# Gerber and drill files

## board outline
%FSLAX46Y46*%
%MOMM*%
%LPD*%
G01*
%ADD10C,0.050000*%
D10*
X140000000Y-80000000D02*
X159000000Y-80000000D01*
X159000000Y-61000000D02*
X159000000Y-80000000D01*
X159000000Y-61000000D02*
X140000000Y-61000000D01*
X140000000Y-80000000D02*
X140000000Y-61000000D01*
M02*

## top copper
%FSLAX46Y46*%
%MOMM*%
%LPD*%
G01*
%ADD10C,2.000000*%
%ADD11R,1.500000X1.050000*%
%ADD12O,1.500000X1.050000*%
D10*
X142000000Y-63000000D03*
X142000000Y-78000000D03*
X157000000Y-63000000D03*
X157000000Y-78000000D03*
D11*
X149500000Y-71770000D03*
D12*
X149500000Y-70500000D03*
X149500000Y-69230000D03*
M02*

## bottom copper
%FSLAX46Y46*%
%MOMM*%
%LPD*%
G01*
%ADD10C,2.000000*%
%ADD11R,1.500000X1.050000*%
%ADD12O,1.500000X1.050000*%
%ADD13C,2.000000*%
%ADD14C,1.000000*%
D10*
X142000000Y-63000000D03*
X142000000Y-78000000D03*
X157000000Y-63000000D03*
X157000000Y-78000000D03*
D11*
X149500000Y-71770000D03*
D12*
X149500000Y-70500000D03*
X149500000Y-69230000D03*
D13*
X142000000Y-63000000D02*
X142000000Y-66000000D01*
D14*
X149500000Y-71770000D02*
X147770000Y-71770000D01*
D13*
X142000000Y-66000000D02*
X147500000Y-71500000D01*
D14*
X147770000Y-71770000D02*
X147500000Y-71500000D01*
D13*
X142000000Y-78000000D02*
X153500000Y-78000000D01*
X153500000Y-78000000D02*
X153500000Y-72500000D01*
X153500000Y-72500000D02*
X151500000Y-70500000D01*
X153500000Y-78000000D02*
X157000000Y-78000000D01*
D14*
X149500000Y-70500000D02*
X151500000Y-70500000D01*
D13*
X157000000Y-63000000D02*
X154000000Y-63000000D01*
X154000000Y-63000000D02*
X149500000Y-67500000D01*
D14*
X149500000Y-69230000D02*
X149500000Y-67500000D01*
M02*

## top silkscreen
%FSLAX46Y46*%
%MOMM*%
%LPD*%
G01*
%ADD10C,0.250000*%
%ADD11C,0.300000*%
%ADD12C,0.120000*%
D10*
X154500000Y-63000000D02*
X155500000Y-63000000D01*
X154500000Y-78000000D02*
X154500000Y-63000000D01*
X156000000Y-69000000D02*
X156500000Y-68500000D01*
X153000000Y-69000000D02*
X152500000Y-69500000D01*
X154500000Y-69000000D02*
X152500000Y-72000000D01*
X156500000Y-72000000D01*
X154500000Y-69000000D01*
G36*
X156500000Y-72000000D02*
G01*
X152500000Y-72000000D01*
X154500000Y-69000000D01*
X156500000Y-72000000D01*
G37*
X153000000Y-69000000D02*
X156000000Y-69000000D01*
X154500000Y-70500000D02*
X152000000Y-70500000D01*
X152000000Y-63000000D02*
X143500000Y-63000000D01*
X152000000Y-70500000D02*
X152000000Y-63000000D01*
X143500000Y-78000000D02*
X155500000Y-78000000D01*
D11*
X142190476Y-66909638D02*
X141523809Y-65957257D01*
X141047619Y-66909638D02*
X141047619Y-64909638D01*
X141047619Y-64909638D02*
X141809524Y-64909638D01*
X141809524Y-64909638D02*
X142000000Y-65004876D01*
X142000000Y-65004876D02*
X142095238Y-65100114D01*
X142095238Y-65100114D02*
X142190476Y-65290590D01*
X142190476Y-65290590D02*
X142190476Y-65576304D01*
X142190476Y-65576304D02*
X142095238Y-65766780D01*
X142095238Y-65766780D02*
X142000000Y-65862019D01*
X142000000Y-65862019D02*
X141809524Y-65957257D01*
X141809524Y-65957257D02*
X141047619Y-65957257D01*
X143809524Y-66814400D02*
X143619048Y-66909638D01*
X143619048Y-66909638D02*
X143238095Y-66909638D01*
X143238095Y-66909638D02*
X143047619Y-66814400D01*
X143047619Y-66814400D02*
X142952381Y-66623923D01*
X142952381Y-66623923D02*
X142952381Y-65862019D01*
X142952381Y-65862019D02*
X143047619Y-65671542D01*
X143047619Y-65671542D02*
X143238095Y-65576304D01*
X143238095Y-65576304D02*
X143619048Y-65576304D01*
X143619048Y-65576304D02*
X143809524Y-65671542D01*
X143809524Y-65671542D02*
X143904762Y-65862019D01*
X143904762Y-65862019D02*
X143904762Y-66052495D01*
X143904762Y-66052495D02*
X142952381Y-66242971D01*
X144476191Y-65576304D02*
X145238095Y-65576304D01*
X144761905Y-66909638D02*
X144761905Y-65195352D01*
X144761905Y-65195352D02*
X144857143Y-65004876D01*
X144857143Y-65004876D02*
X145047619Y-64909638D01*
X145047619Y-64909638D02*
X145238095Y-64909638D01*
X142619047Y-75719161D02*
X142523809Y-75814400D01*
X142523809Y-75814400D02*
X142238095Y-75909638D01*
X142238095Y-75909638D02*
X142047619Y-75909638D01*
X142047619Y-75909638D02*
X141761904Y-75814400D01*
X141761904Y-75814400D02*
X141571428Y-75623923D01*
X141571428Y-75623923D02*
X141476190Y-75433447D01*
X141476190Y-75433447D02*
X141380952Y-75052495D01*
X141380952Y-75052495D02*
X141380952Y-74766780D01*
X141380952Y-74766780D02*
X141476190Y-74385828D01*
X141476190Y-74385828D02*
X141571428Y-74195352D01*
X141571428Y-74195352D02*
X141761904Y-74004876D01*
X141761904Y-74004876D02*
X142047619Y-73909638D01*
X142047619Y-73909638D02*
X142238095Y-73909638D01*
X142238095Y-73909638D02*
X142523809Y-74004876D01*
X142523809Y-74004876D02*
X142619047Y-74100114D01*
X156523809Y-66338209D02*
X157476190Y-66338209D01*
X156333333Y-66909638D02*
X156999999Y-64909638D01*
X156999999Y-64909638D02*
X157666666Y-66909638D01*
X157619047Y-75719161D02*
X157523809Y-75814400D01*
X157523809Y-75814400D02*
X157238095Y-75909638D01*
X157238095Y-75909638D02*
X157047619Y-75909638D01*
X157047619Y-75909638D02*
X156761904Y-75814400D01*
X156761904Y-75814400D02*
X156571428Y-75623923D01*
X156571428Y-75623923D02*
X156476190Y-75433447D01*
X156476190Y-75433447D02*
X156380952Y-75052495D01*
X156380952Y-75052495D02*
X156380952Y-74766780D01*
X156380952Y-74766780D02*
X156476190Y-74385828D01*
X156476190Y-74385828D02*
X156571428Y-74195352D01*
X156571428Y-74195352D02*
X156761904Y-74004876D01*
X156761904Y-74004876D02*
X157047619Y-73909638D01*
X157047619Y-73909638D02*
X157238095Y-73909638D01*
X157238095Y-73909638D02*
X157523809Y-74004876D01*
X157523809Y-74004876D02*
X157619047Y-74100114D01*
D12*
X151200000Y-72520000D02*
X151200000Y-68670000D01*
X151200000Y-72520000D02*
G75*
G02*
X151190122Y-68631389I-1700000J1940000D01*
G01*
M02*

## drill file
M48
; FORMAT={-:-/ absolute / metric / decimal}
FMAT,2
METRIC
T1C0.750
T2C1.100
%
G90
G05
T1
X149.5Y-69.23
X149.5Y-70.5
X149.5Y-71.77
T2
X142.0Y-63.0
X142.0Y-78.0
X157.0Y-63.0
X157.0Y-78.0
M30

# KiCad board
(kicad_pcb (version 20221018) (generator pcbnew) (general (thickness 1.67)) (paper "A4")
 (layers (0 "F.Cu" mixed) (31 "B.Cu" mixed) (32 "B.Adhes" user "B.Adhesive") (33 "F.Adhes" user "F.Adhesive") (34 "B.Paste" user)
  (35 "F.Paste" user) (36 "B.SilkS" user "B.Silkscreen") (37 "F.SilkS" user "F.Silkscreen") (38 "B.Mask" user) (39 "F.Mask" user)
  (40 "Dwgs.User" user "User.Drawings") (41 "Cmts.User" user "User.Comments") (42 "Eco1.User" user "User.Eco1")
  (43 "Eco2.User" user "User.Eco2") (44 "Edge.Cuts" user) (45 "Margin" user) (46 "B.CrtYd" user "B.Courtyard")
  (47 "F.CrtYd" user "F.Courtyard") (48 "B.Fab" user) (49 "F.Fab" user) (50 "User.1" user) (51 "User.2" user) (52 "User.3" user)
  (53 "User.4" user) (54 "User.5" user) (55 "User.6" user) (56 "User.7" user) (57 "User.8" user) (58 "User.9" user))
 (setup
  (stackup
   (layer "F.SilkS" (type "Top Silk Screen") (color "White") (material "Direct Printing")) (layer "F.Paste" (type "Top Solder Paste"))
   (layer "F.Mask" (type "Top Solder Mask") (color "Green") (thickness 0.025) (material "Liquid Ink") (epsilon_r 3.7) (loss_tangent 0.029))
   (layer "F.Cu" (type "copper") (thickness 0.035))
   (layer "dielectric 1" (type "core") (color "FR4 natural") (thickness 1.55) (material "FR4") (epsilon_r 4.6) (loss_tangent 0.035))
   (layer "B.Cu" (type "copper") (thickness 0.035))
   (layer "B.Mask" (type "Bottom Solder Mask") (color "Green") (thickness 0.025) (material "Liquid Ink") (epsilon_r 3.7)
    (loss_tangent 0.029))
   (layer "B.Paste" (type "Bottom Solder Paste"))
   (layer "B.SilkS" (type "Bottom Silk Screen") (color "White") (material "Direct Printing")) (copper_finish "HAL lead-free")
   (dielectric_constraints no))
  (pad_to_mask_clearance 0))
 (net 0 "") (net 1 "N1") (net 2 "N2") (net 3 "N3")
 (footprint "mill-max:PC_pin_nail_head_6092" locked (layer "F.Cu") (at 142 63)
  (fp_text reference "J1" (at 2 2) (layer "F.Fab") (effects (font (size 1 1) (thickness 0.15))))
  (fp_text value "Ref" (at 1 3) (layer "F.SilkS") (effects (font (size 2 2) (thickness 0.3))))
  (pad "1" thru_hole circle locked (at 0 0) (size 2 2) (drill 1.1) (layers "*.Cu" "*.Mask") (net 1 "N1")))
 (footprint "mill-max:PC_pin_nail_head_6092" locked (layer "F.Cu") (at 142 78)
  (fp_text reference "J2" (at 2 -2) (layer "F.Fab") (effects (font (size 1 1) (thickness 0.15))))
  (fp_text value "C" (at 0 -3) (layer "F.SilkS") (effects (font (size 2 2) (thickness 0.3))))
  (pad "1" thru_hole circle locked (at 0 0) (size 2 2) (drill 1.1) (layers "*.Cu" "*.Mask") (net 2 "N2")))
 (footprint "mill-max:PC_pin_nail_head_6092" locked (layer "F.Cu") (at 157 63)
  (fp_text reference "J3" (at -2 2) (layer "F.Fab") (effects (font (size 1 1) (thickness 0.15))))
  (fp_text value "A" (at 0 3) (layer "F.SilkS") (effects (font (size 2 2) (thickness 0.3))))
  (pad "1" thru_hole circle locked (at 0 0) (size 2 2) (drill 1.1) (layers "*.Cu" "*.Mask") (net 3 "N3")))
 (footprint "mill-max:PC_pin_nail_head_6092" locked (layer "F.Cu") (at 157 78)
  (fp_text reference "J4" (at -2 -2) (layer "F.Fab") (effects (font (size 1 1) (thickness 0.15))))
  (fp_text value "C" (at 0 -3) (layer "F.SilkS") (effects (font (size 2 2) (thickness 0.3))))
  (pad "1" thru_hole circle locked (at 0 0) (size 2 2) (drill 1.1) (layers "*.Cu" "*.Mask") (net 2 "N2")))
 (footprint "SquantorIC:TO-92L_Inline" (layer "F.Cu") (at 149.5 70.5 90)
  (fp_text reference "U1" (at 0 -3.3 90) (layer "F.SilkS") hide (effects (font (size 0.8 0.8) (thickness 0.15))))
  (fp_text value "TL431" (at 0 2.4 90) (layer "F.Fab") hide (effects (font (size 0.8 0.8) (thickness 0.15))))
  (fp_line (start -2.02 1.7) (end 1.83 1.7) (stroke (width 0.12) (type solid)) (layer "F.SilkS"))
  (fp_arc (start -2.02 1.7) (mid -0.086552 -2.579449) (end 1.868611 1.690122) (stroke (width 0.12) (type solid)) (layer "F.SilkS"))
  (pad "1" thru_hole rect (at -1.27 0 90) (size 1.05 1.5) (drill 0.75) (layers "*.Cu" "*.Mask") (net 1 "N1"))
  (pad "2" thru_hole oval (at 0 0 90) (size 1.05 1.5) (drill 0.75) (layers "*.Cu" "*.Mask") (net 2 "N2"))
  (pad "3" thru_hole oval (at 1.27 0 90) (size 1.05 1.5) (drill 0.75) (layers "*.Cu" "*.Mask") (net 3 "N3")))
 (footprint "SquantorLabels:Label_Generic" (layer "B.Cu") (at 141.1 69.4 -90)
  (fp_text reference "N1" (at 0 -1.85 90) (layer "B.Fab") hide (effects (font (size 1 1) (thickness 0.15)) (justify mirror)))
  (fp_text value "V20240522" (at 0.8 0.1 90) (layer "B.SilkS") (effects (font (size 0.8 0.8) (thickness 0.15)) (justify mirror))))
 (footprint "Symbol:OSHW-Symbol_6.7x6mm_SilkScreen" (layer "B.Cu") (at 145 70 90)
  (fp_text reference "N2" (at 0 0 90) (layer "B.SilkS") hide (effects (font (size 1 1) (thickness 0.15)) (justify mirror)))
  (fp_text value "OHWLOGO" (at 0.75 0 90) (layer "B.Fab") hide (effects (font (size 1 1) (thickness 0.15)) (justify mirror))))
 (gr_line (start 154.5 63) (end 155.5 63) (stroke (width 0.25) (type default)) (layer "F.SilkS"))
 (gr_line (start 154.5 78) (end 154.5 63) (stroke (width 0.25) (type default)) (layer "F.SilkS"))
 (gr_line (start 156 69) (end 156.5 68.5) (stroke (width 0.25) (type default)) (layer "F.SilkS"))
 (gr_line (start 153 69) (end 152.5 69.5) (stroke (width 0.25) (type default)) (layer "F.SilkS"))
 (gr_poly (pts (xy 154.5 69) (xy 152.5 72) (xy 156.5 72)) (stroke (width 0.25) (type solid)) (fill solid) (layer "F.SilkS"))
 (gr_line (start 153 69) (end 156 69) (stroke (width 0.25) (type default)) (layer "F.SilkS"))
 (gr_line (start 154.5 70.5) (end 152 70.5) (stroke (width 0.25) (type default)) (layer "F.SilkS"))
 (gr_line (start 152 63) (end 143.5 63) (stroke (width 0.25) (type default)) (layer "F.SilkS"))
 (gr_line (start 152 70.5) (end 152 63) (stroke (width 0.25) (type default)) (layer "F.SilkS"))
 (gr_line (start 143.5 78) (end 155.5 78) (stroke (width 0.25) (type default)) (layer "F.SilkS"))
 (gr_line (start 140 80) (end 159 80) (stroke (width 0.05) (type solid)) (layer "Edge.Cuts"))
 (gr_line (start 159 61) (end 159 80) (stroke (width 0.05) (type solid)) (layer "Edge.Cuts"))
 (gr_line (start 159 61) (end 140 61) (stroke (width 0.05) (type solid)) (layer "Edge.Cuts"))
 (gr_line (start 140 80) (end 140 61) (stroke (width 0.05) (type solid)) (layer "Edge.Cuts"))
 (segment (start 142 63) (end 142 66) (width 2) (layer "B.Cu") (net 1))
 (segment (start 149.5 71.77) (end 147.77 71.77) (width 1) (layer "B.Cu") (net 1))
 (segment (start 142 66) (end 147.5 71.5) (width 2) (layer "B.Cu") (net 1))
 (segment (start 147.77 71.77) (end 147.5 71.5) (width 1) (layer "B.Cu") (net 1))
 (segment (start 142 78) (end 153.5 78) (width 2) (layer "B.Cu") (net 2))
 (segment (start 153.5 78) (end 153.5 72.5) (width 2) (layer "B.Cu") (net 2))
 (segment (start 153.5 72.5) (end 151.5 70.5) (width 2) (layer "B.Cu") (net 2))
 (segment (start 153.5 78) (end 157 78) (width 2) (layer "B.Cu") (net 2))
 (segment (start 149.5 70.5) (end 151.5 70.5) (width 1) (layer "B.Cu") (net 2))
 (segment (start 157 63) (end 154 63) (width 2) (layer "B.Cu") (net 3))
 (segment (start 154 63) (end 149.5 67.5) (width 2) (layer "B.Cu") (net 3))
 (segment (start 149.5 69.23) (end 149.5 67.5) (width 1) (layer "B.Cu") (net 3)))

